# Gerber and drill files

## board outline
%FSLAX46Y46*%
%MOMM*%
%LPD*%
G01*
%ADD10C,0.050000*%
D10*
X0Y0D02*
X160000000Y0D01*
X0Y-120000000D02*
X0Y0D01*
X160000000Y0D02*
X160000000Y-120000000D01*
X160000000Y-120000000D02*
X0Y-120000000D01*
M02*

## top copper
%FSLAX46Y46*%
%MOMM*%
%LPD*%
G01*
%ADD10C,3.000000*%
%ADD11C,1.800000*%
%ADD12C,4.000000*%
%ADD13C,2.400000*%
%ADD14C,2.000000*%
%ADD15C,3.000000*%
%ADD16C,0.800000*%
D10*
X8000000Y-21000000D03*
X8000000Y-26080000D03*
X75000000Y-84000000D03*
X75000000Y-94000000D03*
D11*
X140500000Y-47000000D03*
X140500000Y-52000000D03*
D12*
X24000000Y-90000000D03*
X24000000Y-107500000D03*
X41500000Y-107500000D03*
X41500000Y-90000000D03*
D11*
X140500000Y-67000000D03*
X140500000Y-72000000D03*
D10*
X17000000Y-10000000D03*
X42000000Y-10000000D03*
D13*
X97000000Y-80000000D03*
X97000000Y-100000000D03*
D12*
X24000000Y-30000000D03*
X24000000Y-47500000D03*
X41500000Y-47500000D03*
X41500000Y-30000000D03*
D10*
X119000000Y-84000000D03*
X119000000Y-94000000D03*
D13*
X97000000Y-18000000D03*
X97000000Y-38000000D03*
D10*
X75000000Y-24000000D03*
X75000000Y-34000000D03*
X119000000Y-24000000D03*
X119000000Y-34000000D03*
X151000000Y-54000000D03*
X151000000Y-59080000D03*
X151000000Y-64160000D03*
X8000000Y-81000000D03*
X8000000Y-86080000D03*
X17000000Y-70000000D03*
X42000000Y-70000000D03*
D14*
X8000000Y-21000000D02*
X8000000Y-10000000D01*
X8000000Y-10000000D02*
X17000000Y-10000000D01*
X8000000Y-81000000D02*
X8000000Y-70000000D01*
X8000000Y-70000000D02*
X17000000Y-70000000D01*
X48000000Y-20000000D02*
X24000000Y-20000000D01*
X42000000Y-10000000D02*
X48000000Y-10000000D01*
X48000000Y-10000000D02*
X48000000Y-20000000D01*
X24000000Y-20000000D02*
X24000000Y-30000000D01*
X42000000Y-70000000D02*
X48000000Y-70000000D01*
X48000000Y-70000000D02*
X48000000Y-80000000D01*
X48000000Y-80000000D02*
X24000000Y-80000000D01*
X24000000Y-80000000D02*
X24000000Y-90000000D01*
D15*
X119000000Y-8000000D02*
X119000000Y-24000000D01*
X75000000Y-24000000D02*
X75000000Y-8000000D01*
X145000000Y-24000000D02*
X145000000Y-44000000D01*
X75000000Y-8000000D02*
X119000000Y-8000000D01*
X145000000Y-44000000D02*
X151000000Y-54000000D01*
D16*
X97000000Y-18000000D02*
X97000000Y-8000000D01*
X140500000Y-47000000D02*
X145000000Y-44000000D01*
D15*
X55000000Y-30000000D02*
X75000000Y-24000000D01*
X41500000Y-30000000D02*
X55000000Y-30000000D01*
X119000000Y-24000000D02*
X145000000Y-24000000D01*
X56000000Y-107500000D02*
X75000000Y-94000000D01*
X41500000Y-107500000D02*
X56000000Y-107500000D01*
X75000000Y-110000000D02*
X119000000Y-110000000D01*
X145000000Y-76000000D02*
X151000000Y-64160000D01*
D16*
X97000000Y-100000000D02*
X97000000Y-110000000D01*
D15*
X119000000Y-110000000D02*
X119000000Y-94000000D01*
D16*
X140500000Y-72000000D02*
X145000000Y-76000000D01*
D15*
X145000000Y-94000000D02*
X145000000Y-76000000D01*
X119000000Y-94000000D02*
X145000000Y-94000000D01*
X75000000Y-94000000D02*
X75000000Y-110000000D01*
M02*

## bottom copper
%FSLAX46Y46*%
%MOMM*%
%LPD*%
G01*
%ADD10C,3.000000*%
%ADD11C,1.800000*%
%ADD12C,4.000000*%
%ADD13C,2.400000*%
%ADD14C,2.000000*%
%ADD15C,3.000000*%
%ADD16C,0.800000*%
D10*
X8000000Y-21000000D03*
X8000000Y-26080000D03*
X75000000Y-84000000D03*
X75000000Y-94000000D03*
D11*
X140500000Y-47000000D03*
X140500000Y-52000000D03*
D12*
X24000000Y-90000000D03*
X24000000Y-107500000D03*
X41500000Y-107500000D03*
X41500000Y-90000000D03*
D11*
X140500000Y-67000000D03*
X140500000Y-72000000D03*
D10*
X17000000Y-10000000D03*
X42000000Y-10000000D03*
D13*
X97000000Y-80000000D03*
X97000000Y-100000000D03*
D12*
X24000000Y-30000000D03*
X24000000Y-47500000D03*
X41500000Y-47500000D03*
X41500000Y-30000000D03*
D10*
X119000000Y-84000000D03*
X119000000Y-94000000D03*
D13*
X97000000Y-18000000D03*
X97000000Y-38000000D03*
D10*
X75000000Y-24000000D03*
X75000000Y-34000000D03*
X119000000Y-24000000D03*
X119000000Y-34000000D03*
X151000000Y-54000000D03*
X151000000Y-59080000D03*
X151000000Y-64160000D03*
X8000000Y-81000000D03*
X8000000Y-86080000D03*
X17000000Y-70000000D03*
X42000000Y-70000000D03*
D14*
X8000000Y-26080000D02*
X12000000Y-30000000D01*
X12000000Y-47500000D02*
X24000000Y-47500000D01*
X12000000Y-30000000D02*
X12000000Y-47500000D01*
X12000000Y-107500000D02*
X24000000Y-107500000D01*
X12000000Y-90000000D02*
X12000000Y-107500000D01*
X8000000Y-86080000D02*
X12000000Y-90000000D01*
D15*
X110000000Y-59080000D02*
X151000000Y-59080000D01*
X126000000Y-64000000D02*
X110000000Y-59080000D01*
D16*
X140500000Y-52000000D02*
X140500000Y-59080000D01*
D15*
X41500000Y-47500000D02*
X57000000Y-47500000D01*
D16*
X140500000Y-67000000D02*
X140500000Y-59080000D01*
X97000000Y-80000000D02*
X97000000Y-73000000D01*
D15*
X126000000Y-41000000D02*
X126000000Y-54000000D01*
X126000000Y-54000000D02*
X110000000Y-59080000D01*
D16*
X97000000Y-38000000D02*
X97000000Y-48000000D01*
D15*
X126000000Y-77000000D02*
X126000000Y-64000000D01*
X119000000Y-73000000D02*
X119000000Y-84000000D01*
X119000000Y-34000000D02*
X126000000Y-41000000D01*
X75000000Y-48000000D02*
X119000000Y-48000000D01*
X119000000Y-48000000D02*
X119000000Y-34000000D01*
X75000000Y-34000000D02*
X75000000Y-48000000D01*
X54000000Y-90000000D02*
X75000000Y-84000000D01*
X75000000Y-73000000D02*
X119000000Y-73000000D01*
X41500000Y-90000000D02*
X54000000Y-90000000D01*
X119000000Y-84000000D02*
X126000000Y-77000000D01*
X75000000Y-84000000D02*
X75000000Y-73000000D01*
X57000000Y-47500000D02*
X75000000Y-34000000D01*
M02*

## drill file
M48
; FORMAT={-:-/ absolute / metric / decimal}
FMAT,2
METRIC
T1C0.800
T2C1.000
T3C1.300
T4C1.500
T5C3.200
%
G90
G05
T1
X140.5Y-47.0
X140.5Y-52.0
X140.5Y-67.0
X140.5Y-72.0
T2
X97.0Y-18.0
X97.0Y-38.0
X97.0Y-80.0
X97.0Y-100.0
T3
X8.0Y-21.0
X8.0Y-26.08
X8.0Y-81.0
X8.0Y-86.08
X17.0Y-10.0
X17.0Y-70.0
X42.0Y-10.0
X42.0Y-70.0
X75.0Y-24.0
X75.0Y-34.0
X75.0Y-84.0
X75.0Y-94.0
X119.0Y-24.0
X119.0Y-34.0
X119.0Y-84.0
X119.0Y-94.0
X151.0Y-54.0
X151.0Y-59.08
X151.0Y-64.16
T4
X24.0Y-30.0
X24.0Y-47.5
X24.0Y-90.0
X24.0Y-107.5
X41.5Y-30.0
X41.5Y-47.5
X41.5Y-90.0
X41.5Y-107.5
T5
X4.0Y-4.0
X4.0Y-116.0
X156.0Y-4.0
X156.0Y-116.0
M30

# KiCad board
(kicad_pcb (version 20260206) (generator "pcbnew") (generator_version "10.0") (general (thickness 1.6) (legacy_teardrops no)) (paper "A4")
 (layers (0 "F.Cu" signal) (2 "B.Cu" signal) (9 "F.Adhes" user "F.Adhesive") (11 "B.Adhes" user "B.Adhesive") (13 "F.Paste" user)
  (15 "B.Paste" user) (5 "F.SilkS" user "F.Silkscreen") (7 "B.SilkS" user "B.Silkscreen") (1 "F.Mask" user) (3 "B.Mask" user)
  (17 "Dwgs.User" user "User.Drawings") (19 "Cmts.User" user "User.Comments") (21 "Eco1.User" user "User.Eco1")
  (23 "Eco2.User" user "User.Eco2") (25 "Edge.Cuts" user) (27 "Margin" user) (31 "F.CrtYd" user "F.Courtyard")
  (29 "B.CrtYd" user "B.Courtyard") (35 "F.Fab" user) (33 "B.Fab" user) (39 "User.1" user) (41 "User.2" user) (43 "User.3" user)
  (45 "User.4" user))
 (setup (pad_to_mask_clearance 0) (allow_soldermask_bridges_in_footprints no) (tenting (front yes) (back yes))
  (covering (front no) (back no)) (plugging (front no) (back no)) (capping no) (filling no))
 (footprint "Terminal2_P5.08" (layer "F.Cu") (at 8 21 -90)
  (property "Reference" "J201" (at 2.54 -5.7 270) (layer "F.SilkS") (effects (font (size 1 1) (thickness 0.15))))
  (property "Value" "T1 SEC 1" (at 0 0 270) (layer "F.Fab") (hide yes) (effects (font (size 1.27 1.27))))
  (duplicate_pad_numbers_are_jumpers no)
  (pad "1" thru_hole circle (at 0 0 270) (size 3 3) (drill 1.3) (layers "*.Cu" "*.Mask") (remove_unused_layers no) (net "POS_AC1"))
  (pad "2" thru_hole circle (at 5.08 0 270) (size 3 3) (drill 1.3) (layers "*.Cu" "*.Mask") (remove_unused_layers no) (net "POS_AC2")))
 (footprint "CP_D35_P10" (layer "F.Cu") (at 75 84 -90)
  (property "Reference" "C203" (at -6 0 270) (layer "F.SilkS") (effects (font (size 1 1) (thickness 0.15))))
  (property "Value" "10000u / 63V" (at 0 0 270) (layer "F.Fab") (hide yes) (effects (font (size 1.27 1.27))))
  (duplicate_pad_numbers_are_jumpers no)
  (pad "1" thru_hole circle (at 0 0 270) (size 3 3) (drill 1.3) (layers "*.Cu" "*.Mask") (remove_unused_layers no) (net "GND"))
  (pad "2" thru_hole circle (at 10 0 270) (size 3 3) (drill 1.3) (layers "*.Cu" "*.Mask") (remove_unused_layers no) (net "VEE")))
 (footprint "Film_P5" (layer "F.Cu") (at 140.5 47 -90)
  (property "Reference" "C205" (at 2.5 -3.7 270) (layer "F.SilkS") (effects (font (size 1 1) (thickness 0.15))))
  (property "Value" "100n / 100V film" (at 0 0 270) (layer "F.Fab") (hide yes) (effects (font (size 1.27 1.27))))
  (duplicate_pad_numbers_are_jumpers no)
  (pad "1" thru_hole circle (at 0 0 270) (size 1.8 1.8) (drill 0.8) (layers "*.Cu" "*.Mask") (remove_unused_layers no) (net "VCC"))
  (pad "2" thru_hole circle (at 5 0 270) (size 1.8 1.8) (drill 0.8) (layers "*.Cu" "*.Mask") (remove_unused_layers no) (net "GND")))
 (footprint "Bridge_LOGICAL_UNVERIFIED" (layer "F.Cu") (at 24 90)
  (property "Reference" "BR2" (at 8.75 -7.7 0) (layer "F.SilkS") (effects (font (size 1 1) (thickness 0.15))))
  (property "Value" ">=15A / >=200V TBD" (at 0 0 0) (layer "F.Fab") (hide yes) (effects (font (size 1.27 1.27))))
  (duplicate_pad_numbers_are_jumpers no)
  (pad "AC1" thru_hole circle (at 0 0) (size 4 4) (drill 1.5) (layers "*.Cu" "*.Mask") (remove_unused_layers no) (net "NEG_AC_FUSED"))
  (pad "AC2" thru_hole circle (at 0 17.5) (size 4 4) (drill 1.5) (layers "*.Cu" "*.Mask") (remove_unused_layers no) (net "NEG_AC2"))
  (pad "N" thru_hole circle (at 17.5 17.5) (size 4 4) (drill 1.5) (layers "*.Cu" "*.Mask") (remove_unused_layers no) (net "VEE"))
  (pad "P" thru_hole circle (at 17.5 0) (size 4 4) (drill 1.5) (layers "*.Cu" "*.Mask") (remove_unused_layers no) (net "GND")))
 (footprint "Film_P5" (layer "F.Cu") (at 140.5 67 -90)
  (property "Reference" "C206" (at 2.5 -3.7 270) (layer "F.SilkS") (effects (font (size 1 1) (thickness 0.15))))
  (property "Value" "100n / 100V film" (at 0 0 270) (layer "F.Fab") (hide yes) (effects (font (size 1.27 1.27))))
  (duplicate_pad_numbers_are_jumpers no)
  (pad "1" thru_hole circle (at 0 0 270) (size 1.8 1.8) (drill 0.8) (layers "*.Cu" "*.Mask") (remove_unused_layers no) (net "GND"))
  (pad "2" thru_hole circle (at 5 0 270) (size 1.8 1.8) (drill 0.8) (layers "*.Cu" "*.Mask") (remove_unused_layers no) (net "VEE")))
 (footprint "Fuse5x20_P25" (layer "F.Cu") (at 17 10)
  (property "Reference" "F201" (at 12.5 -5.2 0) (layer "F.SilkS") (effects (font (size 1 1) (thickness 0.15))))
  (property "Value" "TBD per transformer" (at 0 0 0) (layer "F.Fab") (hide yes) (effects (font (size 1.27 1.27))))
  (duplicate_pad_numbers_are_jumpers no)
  (pad "1" thru_hole circle (at 0 0) (size 3 3) (drill 1.3) (layers "*.Cu" "*.Mask") (remove_unused_layers no) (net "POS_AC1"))
  (pad "2" thru_hole circle (at 25 0) (size 3 3) (drill 1.3) (layers "*.Cu" "*.Mask") (remove_unused_layers no) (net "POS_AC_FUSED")))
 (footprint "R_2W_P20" (layer "F.Cu") (at 97 80 -90)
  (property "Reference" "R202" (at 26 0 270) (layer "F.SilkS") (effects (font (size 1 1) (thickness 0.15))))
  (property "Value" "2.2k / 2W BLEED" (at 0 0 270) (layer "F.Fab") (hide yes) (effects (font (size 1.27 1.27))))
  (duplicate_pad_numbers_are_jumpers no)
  (pad "1" thru_hole circle (at 0 0 270) (size 2.4 2.4) (drill 1) (layers "*.Cu" "*.Mask") (remove_unused_layers no) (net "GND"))
  (pad "2" thru_hole circle (at 20 0 270) (size 2.4 2.4) (drill 1) (layers "*.Cu" "*.Mask") (remove_unused_layers no) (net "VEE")))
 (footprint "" (layer "F.Cu") (at 156 116)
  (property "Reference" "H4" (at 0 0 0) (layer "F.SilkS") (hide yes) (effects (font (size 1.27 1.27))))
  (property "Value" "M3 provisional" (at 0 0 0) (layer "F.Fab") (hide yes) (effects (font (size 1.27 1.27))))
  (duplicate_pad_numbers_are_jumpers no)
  (pad "" np_thru_hole circle (at 0 0) (size 3.2 3.2) (drill 3.2) (layers "*.Cu" "*.Mask")))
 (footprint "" (layer "F.Cu") (at 156 4)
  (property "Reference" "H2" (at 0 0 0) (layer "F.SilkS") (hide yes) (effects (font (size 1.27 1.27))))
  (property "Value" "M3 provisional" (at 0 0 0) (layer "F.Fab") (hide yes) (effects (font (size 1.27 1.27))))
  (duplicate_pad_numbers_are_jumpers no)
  (pad "" np_thru_hole circle (at 0 0) (size 3.2 3.2) (drill 3.2) (layers "*.Cu" "*.Mask")))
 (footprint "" (layer "F.Cu") (at 4 4)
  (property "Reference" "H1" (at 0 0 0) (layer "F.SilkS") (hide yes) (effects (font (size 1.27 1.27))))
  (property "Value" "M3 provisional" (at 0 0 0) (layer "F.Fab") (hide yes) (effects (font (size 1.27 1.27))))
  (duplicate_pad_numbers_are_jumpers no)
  (pad "" np_thru_hole circle (at 0 0) (size 3.2 3.2) (drill 3.2) (layers "*.Cu" "*.Mask")))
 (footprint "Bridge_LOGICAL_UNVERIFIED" (layer "F.Cu") (at 24 30)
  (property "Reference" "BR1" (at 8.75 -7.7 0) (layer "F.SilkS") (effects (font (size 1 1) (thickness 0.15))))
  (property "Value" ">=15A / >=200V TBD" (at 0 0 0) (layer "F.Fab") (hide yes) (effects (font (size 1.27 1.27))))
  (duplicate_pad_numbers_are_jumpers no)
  (pad "AC1" thru_hole circle (at 0 0) (size 4 4) (drill 1.5) (layers "*.Cu" "*.Mask") (remove_unused_layers no) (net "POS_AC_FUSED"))
  (pad "AC2" thru_hole circle (at 0 17.5) (size 4 4) (drill 1.5) (layers "*.Cu" "*.Mask") (remove_unused_layers no) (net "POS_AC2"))
  (pad "N" thru_hole circle (at 17.5 17.5) (size 4 4) (drill 1.5) (layers "*.Cu" "*.Mask") (remove_unused_layers no) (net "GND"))
  (pad "P" thru_hole circle (at 17.5 0) (size 4 4) (drill 1.5) (layers "*.Cu" "*.Mask") (remove_unused_layers no) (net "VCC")))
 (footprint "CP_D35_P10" (layer "F.Cu") (at 119 84 -90)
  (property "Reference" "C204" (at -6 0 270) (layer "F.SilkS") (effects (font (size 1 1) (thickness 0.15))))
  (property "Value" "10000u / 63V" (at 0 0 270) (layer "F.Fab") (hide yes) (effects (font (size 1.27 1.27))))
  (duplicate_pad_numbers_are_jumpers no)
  (pad "1" thru_hole circle (at 0 0 270) (size 3 3) (drill 1.3) (layers "*.Cu" "*.Mask") (remove_unused_layers no) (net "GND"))
  (pad "2" thru_hole circle (at 10 0 270) (size 3 3) (drill 1.3) (layers "*.Cu" "*.Mask") (remove_unused_layers no) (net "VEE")))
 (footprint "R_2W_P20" (layer "F.Cu") (at 97 18 -90)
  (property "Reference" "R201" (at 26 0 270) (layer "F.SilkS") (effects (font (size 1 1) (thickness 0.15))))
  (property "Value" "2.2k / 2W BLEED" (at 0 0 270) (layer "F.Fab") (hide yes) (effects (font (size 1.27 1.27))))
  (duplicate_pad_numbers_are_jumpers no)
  (pad "1" thru_hole circle (at 0 0 270) (size 2.4 2.4) (drill 1) (layers "*.Cu" "*.Mask") (remove_unused_layers no) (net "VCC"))
  (pad "2" thru_hole circle (at 20 0 270) (size 2.4 2.4) (drill 1) (layers "*.Cu" "*.Mask") (remove_unused_layers no) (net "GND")))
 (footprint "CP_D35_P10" (layer "F.Cu") (at 75 24 -90)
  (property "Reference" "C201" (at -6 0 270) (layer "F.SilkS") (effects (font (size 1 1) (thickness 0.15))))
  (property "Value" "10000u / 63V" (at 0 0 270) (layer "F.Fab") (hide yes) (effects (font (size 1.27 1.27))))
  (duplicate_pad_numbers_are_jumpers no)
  (pad "1" thru_hole circle (at 0 0 270) (size 3 3) (drill 1.3) (layers "*.Cu" "*.Mask") (remove_unused_layers no) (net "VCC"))
  (pad "2" thru_hole circle (at 10 0 270) (size 3 3) (drill 1.3) (layers "*.Cu" "*.Mask") (remove_unused_layers no) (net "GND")))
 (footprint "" (layer "F.Cu") (at 4 116)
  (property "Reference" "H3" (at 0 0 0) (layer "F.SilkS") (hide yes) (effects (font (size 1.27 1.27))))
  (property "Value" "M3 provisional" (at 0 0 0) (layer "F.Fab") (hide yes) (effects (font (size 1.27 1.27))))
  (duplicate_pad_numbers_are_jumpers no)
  (pad "" np_thru_hole circle (at 0 0) (size 3.2 3.2) (drill 3.2) (layers "*.Cu" "*.Mask")))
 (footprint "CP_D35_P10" (layer "F.Cu") (at 119 24 -90)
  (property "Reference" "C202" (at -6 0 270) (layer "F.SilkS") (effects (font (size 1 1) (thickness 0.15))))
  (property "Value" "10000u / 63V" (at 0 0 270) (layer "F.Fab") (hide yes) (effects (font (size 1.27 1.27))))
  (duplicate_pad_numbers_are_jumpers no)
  (pad "1" thru_hole circle (at 0 0 270) (size 3 3) (drill 1.3) (layers "*.Cu" "*.Mask") (remove_unused_layers no) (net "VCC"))
  (pad "2" thru_hole circle (at 10 0 270) (size 3 3) (drill 1.3) (layers "*.Cu" "*.Mask") (remove_unused_layers no) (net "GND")))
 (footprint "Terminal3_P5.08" (layer "F.Cu") (at 151 54 -90)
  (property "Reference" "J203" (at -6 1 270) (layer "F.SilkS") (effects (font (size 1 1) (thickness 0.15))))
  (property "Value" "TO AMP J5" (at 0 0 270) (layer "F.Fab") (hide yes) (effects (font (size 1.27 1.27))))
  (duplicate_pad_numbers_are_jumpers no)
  (pad "1" thru_hole circle (at 0 0 270) (size 3 3) (drill 1.3) (layers "*.Cu" "*.Mask") (remove_unused_layers no) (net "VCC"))
  (pad "2" thru_hole circle (at 5.08 0 270) (size 3 3) (drill 1.3) (layers "*.Cu" "*.Mask") (remove_unused_layers no) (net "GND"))
  (pad "3" thru_hole circle (at 10.16 0 270) (size 3 3) (drill 1.3) (layers "*.Cu" "*.Mask") (remove_unused_layers no) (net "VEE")))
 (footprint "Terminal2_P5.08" (layer "F.Cu") (at 8 81 -90)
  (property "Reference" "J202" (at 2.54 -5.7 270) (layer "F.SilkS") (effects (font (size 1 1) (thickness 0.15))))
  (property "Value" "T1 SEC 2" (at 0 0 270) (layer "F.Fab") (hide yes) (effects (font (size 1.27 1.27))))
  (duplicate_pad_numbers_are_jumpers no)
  (pad "1" thru_hole circle (at 0 0 270) (size 3 3) (drill 1.3) (layers "*.Cu" "*.Mask") (remove_unused_layers no) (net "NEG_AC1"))
  (pad "2" thru_hole circle (at 5.08 0 270) (size 3 3) (drill 1.3) (layers "*.Cu" "*.Mask") (remove_unused_layers no) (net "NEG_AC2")))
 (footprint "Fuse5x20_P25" (layer "F.Cu") (at 17 70)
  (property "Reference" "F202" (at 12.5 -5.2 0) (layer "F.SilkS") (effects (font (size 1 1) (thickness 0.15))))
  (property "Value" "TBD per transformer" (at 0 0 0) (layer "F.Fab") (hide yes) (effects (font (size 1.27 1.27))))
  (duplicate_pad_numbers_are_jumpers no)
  (pad "1" thru_hole circle (at 0 0) (size 3 3) (drill 1.3) (layers "*.Cu" "*.Mask") (remove_unused_layers no) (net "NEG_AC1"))
  (pad "2" thru_hole circle (at 25 0) (size 3 3) (drill 1.3) (layers "*.Cu" "*.Mask") (remove_unused_layers no) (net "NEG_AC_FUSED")))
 (gr_line (start 0 0) (end 160 0) (stroke (width 0.05) (type default)) (layer "Edge.Cuts"))
 (gr_line (start 0 120) (end 0 0) (stroke (width 0.05) (type default)) (layer "Edge.Cuts"))
 (gr_line (start 160 0) (end 160 120) (stroke (width 0.05) (type default)) (layer "Edge.Cuts"))
 (gr_line (start 160 120) (end 0 120) (stroke (width 0.05) (type default)) (layer "Edge.Cuts"))
 (segment (start 8 21) (end 8 10) (width 2) (layer "F.Cu") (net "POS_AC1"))
 (segment (start 8 10) (end 17 10) (width 2) (layer "F.Cu") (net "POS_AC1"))
 (segment (start 8 26.08) (end 12 30) (width 2) (layer "B.Cu") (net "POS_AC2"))
 (segment (start 12 47.5) (end 24 47.5) (width 2) (layer "B.Cu") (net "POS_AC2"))
 (segment (start 12 30) (end 12 47.5) (width 2) (layer "B.Cu") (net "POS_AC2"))
 (segment (start 8 81) (end 8 70) (width 2) (layer "F.Cu") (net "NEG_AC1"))
 (segment (start 8 70) (end 17 70) (width 2) (layer "F.Cu") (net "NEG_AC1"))
 (segment (start 12 107.5) (end 24 107.5) (width 2) (layer "B.Cu") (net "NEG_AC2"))
 (segment (start 12 90) (end 12 107.5) (width 2) (layer "B.Cu") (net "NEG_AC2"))
 (segment (start 8 86.08) (end 12 90) (width 2) (layer "B.Cu") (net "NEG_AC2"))
 (segment (start 48 20) (end 24 20) (width 2) (layer "F.Cu") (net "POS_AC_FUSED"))
 (segment (start 42 10) (end 48 10) (width 2) (layer "F.Cu") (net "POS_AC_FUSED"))
 (segment (start 48 10) (end 48 20) (width 2) (layer "F.Cu") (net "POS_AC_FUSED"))
 (segment (start 24 20) (end 24 30) (width 2) (layer "F.Cu") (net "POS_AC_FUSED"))
 (segment (start 42 70) (end 48 70) (width 2) (layer "F.Cu") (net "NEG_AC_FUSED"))
 (segment (start 48 70) (end 48 80) (width 2) (layer "F.Cu") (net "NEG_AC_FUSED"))
 (segment (start 48 80) (end 24 80) (width 2) (layer "F.Cu") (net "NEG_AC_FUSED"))
 (segment (start 24 80) (end 24 90) (width 2) (layer "F.Cu") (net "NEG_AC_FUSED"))
 (segment (start 110 59.08) (end 151 59.08) (width 3) (layer "B.Cu") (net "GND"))
 (segment (start 126 64) (end 110 59.08) (width 3) (layer "B.Cu") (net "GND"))
 (segment (start 140.5 52) (end 140.5 59.08) (width 0.8) (layer "B.Cu") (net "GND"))
 (segment (start 41.5 47.5) (end 57 47.5) (width 3) (layer "B.Cu") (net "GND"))
 (segment (start 140.5 67) (end 140.5 59.08) (width 0.8) (layer "B.Cu") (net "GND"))
 (segment (start 97 80) (end 97 73) (width 0.8) (layer "B.Cu") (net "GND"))
 (segment (start 126 41) (end 126 54) (width 3) (layer "B.Cu") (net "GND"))
 (segment (start 126 54) (end 110 59.08) (width 3) (layer "B.Cu") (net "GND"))
 (segment (start 97 38) (end 97 48) (width 0.8) (layer "B.Cu") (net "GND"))
 (segment (start 126 77) (end 126 64) (width 3) (layer "B.Cu") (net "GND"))
 (segment (start 119 73) (end 119 84) (width 3) (layer "B.Cu") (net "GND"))
 (segment (start 119 34) (end 126 41) (width 3) (layer "B.Cu") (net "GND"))
 (segment (start 75 48) (end 119 48) (width 3) (layer "B.Cu") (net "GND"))
 (segment (start 119 48) (end 119 34) (width 3) (layer "B.Cu") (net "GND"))
 (segment (start 75 34) (end 75 48) (width 3) (layer "B.Cu") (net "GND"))
 (segment (start 54 90) (end 75 84) (width 3) (layer "B.Cu") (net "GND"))
 (segment (start 75 73) (end 119 73) (width 3) (layer "B.Cu") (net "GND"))
 (segment (start 41.5 90) (end 54 90) (width 3) (layer "B.Cu") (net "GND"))
 (segment (start 119 84) (end 126 77) (width 3) (layer "B.Cu") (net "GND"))
 (segment (start 75 84) (end 75 73) (width 3) (layer "B.Cu") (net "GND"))
 (segment (start 57 47.5) (end 75 34) (width 3) (layer "B.Cu") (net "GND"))
 (segment (start 119 8) (end 119 24) (width 3) (layer "F.Cu") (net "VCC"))
 (segment (start 75 24) (end 75 8) (width 3) (layer "F.Cu") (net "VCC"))
 (segment (start 145 24) (end 145 44) (width 3) (layer "F.Cu") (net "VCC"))
 (segment (start 75 8) (end 119 8) (width 3) (layer "F.Cu") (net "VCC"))
 (segment (start 145 44) (end 151 54) (width 3) (layer "F.Cu") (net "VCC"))
 (segment (start 97 18) (end 97 8) (width 0.8) (layer "F.Cu") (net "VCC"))
 (segment (start 140.5 47) (end 145 44) (width 0.8) (layer "F.Cu") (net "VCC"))
 (segment (start 55 30) (end 75 24) (width 3) (layer "F.Cu") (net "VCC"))
 (segment (start 41.5 30) (end 55 30) (width 3) (layer "F.Cu") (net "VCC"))
 (segment (start 119 24) (end 145 24) (width 3) (layer "F.Cu") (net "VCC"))
 (segment (start 56 107.5) (end 75 94) (width 3) (layer "F.Cu") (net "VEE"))
 (segment (start 41.5 107.5) (end 56 107.5) (width 3) (layer "F.Cu") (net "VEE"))
 (segment (start 75 110) (end 119 110) (width 3) (layer "F.Cu") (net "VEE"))
 (segment (start 145 76) (end 151 64.16) (width 3) (layer "F.Cu") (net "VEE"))
 (segment (start 97 100) (end 97 110) (width 0.8) (layer "F.Cu") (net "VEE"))
 (segment (start 119 110) (end 119 94) (width 3) (layer "F.Cu") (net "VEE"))
 (segment (start 140.5 72) (end 145 76) (width 0.8) (layer "F.Cu") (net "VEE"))
 (segment (start 145 94) (end 145 76) (width 3) (layer "F.Cu") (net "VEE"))
 (segment (start 119 94) (end 145 94) (width 3) (layer "F.Cu") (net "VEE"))
 (segment (start 75 94) (end 75 110) (width 3) (layer "F.Cu") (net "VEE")))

